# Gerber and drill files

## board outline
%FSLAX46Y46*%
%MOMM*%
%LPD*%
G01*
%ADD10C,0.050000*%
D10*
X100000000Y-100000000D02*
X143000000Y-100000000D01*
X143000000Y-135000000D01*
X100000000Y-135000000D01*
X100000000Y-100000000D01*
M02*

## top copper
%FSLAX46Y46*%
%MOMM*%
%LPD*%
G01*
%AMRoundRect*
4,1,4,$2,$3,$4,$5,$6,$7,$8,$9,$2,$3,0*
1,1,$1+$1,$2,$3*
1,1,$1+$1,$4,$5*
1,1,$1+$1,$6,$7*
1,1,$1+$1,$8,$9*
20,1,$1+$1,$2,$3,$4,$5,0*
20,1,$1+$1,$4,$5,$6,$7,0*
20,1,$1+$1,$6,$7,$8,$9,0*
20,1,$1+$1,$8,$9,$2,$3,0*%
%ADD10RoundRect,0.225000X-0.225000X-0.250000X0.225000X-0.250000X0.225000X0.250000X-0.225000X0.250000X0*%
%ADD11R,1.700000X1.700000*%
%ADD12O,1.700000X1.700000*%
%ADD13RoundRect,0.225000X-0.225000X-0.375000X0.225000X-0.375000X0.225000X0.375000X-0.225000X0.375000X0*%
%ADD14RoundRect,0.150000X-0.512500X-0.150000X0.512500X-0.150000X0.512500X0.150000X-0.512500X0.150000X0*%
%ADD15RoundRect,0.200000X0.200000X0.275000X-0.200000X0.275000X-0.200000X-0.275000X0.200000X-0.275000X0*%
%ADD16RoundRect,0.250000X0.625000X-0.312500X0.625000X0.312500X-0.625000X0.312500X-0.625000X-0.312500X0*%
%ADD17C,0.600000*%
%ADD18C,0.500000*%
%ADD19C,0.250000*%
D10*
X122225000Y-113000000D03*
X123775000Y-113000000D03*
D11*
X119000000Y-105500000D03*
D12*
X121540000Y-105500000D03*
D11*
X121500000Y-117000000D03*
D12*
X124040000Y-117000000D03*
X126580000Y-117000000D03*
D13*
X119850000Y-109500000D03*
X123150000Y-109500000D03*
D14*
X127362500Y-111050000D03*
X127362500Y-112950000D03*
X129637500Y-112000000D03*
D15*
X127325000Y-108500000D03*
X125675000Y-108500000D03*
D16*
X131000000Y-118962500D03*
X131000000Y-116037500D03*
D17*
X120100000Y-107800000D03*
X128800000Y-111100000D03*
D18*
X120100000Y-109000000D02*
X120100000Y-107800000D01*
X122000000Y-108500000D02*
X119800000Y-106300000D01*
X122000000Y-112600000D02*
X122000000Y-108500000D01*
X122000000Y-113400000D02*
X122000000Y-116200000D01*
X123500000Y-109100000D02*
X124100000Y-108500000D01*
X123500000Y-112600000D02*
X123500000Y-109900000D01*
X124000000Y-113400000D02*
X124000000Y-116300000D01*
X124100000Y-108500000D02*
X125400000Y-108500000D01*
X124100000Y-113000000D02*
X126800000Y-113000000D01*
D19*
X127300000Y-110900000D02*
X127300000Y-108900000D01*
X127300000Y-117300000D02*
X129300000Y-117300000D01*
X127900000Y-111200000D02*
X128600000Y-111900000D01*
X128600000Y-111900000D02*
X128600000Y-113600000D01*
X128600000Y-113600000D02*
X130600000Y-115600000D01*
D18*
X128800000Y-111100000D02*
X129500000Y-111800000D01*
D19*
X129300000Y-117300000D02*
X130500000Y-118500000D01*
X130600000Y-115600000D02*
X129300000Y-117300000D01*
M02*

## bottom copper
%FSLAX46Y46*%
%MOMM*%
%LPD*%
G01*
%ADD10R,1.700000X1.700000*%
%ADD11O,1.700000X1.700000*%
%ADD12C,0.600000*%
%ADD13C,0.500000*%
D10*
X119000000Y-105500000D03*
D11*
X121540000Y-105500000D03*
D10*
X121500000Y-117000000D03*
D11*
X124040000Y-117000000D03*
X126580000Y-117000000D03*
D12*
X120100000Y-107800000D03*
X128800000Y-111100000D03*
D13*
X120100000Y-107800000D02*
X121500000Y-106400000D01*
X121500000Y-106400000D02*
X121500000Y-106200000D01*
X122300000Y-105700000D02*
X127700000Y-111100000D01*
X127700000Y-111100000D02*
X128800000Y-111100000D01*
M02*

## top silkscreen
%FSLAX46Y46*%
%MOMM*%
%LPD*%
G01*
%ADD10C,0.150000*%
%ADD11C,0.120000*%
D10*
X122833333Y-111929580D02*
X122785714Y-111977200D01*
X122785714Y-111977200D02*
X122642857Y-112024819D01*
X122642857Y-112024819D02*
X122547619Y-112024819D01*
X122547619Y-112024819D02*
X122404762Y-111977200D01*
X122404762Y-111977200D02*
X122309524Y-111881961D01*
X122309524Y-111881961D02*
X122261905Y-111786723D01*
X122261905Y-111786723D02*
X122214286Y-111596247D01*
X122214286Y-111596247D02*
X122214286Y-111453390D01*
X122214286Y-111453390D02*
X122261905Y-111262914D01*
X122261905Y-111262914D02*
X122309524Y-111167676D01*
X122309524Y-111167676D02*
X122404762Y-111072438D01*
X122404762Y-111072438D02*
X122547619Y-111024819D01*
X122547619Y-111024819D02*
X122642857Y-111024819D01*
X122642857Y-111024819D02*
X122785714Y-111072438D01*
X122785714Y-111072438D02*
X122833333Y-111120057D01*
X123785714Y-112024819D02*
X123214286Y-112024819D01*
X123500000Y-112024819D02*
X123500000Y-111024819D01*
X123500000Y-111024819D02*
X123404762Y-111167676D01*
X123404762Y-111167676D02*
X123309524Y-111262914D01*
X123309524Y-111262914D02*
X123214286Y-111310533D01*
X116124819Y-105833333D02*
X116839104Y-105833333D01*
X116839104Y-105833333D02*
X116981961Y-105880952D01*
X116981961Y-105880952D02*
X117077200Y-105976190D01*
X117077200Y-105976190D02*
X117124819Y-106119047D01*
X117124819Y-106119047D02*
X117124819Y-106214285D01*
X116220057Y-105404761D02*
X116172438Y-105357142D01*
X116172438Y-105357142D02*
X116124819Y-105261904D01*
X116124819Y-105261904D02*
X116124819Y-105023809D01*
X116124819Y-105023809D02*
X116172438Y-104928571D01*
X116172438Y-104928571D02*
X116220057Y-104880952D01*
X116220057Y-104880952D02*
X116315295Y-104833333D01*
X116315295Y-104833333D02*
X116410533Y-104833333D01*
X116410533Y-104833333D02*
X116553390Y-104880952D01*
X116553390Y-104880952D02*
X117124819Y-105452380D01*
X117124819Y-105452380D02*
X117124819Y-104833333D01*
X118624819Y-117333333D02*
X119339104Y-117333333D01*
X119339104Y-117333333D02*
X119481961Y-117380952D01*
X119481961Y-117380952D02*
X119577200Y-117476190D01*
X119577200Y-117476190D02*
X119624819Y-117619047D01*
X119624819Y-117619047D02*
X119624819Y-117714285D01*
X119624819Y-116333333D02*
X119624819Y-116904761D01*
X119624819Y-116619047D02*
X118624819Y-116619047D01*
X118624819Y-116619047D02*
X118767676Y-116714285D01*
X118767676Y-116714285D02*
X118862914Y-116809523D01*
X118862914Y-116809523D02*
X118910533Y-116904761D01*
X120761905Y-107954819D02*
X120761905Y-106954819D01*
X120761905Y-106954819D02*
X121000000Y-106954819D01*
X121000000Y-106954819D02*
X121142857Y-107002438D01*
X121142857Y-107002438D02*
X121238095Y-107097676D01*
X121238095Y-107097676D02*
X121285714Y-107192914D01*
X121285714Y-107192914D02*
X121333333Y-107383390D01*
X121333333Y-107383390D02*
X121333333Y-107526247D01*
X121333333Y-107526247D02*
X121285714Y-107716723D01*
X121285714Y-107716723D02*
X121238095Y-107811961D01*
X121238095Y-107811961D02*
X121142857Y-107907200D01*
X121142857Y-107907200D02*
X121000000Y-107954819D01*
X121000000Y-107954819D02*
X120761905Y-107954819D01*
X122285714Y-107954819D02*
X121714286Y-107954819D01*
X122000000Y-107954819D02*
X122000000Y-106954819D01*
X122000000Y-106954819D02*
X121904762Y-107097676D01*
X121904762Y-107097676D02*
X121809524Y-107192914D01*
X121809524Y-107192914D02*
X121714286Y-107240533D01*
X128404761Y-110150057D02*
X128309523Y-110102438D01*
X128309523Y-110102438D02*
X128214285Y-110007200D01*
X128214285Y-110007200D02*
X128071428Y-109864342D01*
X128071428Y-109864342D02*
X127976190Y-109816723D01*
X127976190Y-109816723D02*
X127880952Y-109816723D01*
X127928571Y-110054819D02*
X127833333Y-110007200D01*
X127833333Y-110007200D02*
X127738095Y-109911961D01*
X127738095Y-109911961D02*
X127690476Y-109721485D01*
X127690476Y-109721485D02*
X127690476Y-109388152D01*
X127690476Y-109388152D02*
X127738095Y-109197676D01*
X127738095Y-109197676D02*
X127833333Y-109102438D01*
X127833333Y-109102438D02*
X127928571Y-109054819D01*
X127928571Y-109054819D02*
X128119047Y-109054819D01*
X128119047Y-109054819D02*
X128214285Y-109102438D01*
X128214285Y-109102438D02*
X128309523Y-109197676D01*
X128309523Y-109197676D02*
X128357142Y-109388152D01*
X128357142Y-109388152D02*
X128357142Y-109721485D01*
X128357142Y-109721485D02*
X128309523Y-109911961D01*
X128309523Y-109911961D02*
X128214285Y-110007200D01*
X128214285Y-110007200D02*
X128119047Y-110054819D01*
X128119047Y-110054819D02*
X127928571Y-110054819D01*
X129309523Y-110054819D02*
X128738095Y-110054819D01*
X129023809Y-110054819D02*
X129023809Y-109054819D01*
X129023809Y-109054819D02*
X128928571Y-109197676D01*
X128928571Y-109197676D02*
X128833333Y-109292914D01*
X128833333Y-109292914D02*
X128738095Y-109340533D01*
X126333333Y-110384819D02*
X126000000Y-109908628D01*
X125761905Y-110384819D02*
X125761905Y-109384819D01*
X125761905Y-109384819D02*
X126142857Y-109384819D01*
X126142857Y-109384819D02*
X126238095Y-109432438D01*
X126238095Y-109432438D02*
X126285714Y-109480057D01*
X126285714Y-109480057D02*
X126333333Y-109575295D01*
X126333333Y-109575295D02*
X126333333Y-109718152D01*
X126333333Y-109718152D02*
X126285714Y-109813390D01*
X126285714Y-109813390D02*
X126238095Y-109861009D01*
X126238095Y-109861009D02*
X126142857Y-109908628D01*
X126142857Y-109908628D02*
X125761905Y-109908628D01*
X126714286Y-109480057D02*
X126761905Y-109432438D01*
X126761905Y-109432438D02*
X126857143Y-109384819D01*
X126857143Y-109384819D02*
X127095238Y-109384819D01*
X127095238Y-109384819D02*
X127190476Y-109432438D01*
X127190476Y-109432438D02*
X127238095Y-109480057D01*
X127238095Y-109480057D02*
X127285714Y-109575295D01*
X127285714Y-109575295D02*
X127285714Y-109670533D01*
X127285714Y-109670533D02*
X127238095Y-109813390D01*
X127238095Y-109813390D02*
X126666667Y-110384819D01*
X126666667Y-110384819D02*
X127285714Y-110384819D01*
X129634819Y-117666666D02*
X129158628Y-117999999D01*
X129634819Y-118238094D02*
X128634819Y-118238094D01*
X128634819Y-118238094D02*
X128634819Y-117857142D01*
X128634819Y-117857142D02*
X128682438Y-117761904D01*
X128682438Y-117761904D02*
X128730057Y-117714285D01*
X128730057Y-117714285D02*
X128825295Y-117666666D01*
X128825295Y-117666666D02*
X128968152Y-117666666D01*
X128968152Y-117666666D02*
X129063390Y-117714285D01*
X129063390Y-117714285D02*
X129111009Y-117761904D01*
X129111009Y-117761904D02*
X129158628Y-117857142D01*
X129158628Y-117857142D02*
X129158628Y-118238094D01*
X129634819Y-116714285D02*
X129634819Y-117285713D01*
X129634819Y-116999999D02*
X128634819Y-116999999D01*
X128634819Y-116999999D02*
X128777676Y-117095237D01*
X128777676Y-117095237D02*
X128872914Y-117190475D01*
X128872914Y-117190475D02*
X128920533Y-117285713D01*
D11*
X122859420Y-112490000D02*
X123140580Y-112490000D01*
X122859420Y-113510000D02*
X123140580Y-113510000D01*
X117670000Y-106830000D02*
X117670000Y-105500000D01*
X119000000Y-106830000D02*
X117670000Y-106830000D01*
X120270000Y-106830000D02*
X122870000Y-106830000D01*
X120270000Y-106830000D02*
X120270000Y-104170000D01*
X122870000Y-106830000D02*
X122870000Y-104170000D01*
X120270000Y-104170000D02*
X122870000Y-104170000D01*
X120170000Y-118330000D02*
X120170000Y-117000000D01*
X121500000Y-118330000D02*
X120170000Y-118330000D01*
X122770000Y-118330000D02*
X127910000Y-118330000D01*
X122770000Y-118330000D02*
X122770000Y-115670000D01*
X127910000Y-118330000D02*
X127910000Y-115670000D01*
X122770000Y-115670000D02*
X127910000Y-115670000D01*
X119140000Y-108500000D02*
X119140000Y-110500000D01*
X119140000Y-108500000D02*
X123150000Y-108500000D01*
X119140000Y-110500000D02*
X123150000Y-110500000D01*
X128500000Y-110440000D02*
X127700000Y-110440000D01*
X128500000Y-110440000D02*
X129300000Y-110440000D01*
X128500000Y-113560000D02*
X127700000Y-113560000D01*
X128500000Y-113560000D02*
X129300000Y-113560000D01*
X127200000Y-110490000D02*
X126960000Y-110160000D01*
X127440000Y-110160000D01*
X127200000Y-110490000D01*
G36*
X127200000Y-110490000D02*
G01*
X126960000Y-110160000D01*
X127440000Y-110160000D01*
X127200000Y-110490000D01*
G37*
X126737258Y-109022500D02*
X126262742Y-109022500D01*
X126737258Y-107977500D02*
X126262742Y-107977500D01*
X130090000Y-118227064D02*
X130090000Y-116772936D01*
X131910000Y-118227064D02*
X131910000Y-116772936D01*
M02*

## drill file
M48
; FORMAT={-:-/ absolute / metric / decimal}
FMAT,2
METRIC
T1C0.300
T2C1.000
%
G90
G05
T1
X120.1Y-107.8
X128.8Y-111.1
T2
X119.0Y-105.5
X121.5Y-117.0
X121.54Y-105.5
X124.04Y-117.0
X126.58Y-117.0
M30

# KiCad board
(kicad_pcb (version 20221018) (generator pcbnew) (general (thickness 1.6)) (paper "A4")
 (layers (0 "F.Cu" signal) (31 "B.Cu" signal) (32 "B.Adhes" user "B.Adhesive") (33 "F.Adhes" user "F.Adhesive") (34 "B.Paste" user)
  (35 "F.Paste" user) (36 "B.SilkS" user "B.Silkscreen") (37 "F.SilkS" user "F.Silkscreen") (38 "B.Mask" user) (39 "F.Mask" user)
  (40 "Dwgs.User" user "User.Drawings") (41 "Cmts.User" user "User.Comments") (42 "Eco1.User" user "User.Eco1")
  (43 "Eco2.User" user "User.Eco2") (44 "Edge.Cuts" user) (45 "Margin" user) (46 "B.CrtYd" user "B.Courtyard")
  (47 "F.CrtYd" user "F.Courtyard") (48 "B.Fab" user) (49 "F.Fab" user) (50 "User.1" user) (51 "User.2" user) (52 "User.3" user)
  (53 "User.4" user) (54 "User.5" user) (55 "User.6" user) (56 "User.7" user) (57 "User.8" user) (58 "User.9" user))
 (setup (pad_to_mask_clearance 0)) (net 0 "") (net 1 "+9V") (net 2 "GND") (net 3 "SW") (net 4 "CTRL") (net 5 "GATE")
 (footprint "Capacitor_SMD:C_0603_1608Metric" (layer "F.Cu") (at 123 113)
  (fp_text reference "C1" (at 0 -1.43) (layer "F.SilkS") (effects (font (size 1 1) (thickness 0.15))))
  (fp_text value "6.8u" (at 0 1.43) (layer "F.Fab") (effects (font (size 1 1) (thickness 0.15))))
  (fp_line (start -0.14058 -0.51) (end 0.14058 -0.51) (stroke (width 0.12) (type solid)) (layer "F.SilkS"))
  (fp_line (start -0.14058 0.51) (end 0.14058 0.51) (stroke (width 0.12) (type solid)) (layer "F.SilkS"))
  (pad "1" smd roundrect (at -0.775 0) (size 0.9 0.95) (layers "F.Cu" "F.Paste" "F.Mask") (roundrect_rratio 0.25) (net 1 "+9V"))
  (pad "2" smd roundrect (at 0.775 0) (size 0.9 0.95) (layers "F.Cu" "F.Paste" "F.Mask") (roundrect_rratio 0.25) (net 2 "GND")))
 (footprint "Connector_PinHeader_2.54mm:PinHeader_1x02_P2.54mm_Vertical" (layer "F.Cu") (at 119 105.5 90)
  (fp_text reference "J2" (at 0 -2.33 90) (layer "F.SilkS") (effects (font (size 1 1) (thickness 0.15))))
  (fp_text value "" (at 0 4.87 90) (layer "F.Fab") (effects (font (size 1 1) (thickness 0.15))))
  (fp_line (start -1.33 -1.33) (end 0 -1.33) (stroke (width 0.12) (type solid)) (layer "F.SilkS"))
  (fp_line (start -1.33 0) (end -1.33 -1.33) (stroke (width 0.12) (type solid)) (layer "F.SilkS"))
  (fp_line (start -1.33 1.27) (end -1.33 3.87) (stroke (width 0.12) (type solid)) (layer "F.SilkS"))
  (fp_line (start -1.33 1.27) (end 1.33 1.27) (stroke (width 0.12) (type solid)) (layer "F.SilkS"))
  (fp_line (start -1.33 3.87) (end 1.33 3.87) (stroke (width 0.12) (type solid)) (layer "F.SilkS"))
  (fp_line (start 1.33 1.27) (end 1.33 3.87) (stroke (width 0.12) (type solid)) (layer "F.SilkS"))
  (pad "1" thru_hole rect (at 0 0 90) (size 1.7 1.7) (drill 1) (layers "*.Cu" "*.Mask") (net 1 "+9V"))
  (pad "2" thru_hole oval (at 0 2.54 90) (size 1.7 1.7) (drill 1) (layers "*.Cu" "*.Mask") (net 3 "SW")))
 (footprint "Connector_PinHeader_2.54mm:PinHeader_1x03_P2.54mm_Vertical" (layer "F.Cu") (at 121.5 117 90)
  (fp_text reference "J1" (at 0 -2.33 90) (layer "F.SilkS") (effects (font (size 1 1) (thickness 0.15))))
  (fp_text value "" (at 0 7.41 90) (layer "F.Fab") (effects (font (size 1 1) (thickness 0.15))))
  (fp_line (start -1.33 -1.33) (end 0 -1.33) (stroke (width 0.12) (type solid)) (layer "F.SilkS"))
  (fp_line (start -1.33 0) (end -1.33 -1.33) (stroke (width 0.12) (type solid)) (layer "F.SilkS"))
  (fp_line (start -1.33 1.27) (end -1.33 6.41) (stroke (width 0.12) (type solid)) (layer "F.SilkS"))
  (fp_line (start -1.33 1.27) (end 1.33 1.27) (stroke (width 0.12) (type solid)) (layer "F.SilkS"))
  (fp_line (start -1.33 6.41) (end 1.33 6.41) (stroke (width 0.12) (type solid)) (layer "F.SilkS"))
  (fp_line (start 1.33 1.27) (end 1.33 6.41) (stroke (width 0.12) (type solid)) (layer "F.SilkS"))
  (pad "1" thru_hole rect (at 0 0 90) (size 1.7 1.7) (drill 1) (layers "*.Cu" "*.Mask") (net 1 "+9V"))
  (pad "2" thru_hole oval (at 0 2.54 90) (size 1.7 1.7) (drill 1) (layers "*.Cu" "*.Mask") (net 2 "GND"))
  (pad "3" thru_hole oval (at 0 5.08 90) (size 1.7 1.7) (drill 1) (layers "*.Cu" "*.Mask") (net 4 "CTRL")))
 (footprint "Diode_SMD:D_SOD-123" (layer "F.Cu") (at 121.5 109.5)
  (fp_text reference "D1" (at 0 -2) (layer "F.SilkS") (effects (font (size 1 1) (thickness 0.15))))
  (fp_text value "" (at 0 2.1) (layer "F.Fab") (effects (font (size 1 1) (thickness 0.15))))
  (fp_line (start -2.36 -1) (end -2.36 1) (stroke (width 0.12) (type solid)) (layer "F.SilkS"))
  (fp_line (start -2.36 -1) (end 1.65 -1) (stroke (width 0.12) (type solid)) (layer "F.SilkS"))
  (fp_line (start -2.36 1) (end 1.65 1) (stroke (width 0.12) (type solid)) (layer "F.SilkS"))
  (pad "1" smd roundrect (at -1.65 0) (size 0.9 1.2) (layers "F.Cu" "F.Paste" "F.Mask") (roundrect_rratio 0.25) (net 3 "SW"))
  (pad "2" smd roundrect (at 1.65 0) (size 0.9 1.2) (layers "F.Cu" "F.Paste" "F.Mask") (roundrect_rratio 0.25) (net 2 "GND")))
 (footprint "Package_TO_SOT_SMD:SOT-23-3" (layer "F.Cu") (at 128.5 112)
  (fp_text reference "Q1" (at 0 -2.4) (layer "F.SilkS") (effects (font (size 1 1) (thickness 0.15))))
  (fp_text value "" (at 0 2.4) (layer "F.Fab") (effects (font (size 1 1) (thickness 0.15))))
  (fp_line (start 0 -1.56) (end -0.8 -1.56) (stroke (width 0.12) (type solid)) (layer "F.SilkS"))
  (fp_line (start 0 -1.56) (end 0.8 -1.56) (stroke (width 0.12) (type solid)) (layer "F.SilkS"))
  (fp_line (start 0 1.56) (end -0.8 1.56) (stroke (width 0.12) (type solid)) (layer "F.SilkS"))
  (fp_line (start 0 1.56) (end 0.8 1.56) (stroke (width 0.12) (type solid)) (layer "F.SilkS"))
  (fp_poly
   (pts (xy -1.3 -1.51) (xy -1.54 -1.84) (xy -1.06 -1.84) (xy -1.3 -1.51)) (stroke (width 0.12) (type solid)) (fill solid) (layer "F.SilkS"))
  (pad "1" smd roundrect (at -1.1375 -0.95) (size 1.325 0.6) (layers "F.Cu" "F.Paste" "F.Mask") (roundrect_rratio 0.25) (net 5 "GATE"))
  (pad "2" smd roundrect (at -1.1375 0.95) (size 1.325 0.6) (layers "F.Cu" "F.Paste" "F.Mask") (roundrect_rratio 0.25) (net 2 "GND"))
  (pad "3" smd roundrect (at 1.1375 0) (size 1.325 0.6) (layers "F.Cu" "F.Paste" "F.Mask") (roundrect_rratio 0.25) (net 3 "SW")))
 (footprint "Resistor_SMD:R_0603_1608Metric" (layer "F.Cu") (at 126.5 108.5 180)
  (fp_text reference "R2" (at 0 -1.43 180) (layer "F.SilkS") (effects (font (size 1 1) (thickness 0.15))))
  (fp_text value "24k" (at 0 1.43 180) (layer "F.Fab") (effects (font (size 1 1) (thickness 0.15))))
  (fp_line (start -0.237258 -0.5225) (end 0.237258 -0.5225) (stroke (width 0.12) (type solid)) (layer "F.SilkS"))
  (fp_line (start -0.237258 0.5225) (end 0.237258 0.5225) (stroke (width 0.12) (type solid)) (layer "F.SilkS"))
  (pad "1" smd roundrect (at -0.825 0 180) (size 0.8 0.95) (layers "F.Cu" "F.Paste" "F.Mask") (roundrect_rratio 0.25) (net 5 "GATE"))
  (pad "2" smd roundrect (at 0.825 0 180) (size 0.8 0.95) (layers "F.Cu" "F.Paste" "F.Mask") (roundrect_rratio 0.25) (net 2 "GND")))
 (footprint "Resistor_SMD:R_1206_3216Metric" (layer "F.Cu") (at 131 117.5 90)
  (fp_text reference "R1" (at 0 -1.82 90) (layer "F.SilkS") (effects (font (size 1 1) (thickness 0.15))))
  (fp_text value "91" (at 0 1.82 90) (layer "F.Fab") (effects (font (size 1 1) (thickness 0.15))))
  (fp_line (start -0.727064 -0.91) (end 0.727064 -0.91) (stroke (width 0.12) (type solid)) (layer "F.SilkS"))
  (fp_line (start -0.727064 0.91) (end 0.727064 0.91) (stroke (width 0.12) (type solid)) (layer "F.SilkS"))
  (pad "1" smd roundrect (at -1.4625 0 90) (size 1.125 1.75) (layers "F.Cu" "F.Paste" "F.Mask") (roundrect_rratio 0.222222) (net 4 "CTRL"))
  (pad "2" smd roundrect (at 1.4625 0 90) (size 1.125 1.75) (layers "F.Cu" "F.Paste" "F.Mask") (roundrect_rratio 0.222222) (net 5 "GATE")))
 (gr_rect (start 100 100) (end 143 135) (stroke (width 0.05) (type default)) (fill none) (layer "Edge.Cuts"))
 (segment (start 120.1 109) (end 120.1 107.8) (width 0.5) (layer "F.Cu") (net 3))
 (segment (start 122 108.5) (end 119.8 106.3) (width 0.5) (layer "F.Cu") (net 1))
 (segment (start 122 112.6) (end 122 108.5) (width 0.5) (layer "F.Cu") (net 1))
 (segment (start 122 113.4) (end 122 116.2) (width 0.5) (layer "F.Cu") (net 1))
 (segment (start 123.5 109.1) (end 124.1 108.5) (width 0.5) (layer "F.Cu") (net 2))
 (segment (start 123.5 112.6) (end 123.5 109.9) (width 0.5) (layer "F.Cu") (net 2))
 (segment (start 124 113.4) (end 124 116.3) (width 0.5) (layer "F.Cu") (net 2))
 (segment (start 124.1 108.5) (end 125.4 108.5) (width 0.5) (layer "F.Cu") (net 2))
 (segment (start 124.1 113) (end 126.8 113) (width 0.5) (layer "F.Cu") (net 2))
 (segment (start 127.3 110.9) (end 127.3 108.9) (width 0.25) (layer "F.Cu") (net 5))
 (segment (start 127.3 117.3) (end 129.3 117.3) (width 0.25) (layer "F.Cu") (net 4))
 (segment (start 127.9 111.2) (end 128.6 111.9) (width 0.25) (layer "F.Cu") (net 5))
 (segment (start 128.6 111.9) (end 128.6 113.6) (width 0.25) (layer "F.Cu") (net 5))
 (segment (start 128.6 113.6) (end 130.6 115.6) (width 0.25) (layer "F.Cu") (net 5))
 (segment (start 128.8 111.1) (end 129.5 111.8) (width 0.5) (layer "F.Cu") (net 3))
 (segment (start 129.3 117.3) (end 130.5 118.5) (width 0.25) (layer "F.Cu") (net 4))
 (segment (start 130.6 115.6) (end 129.3 117.3) (width 0.25) (layer "F.Cu") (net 5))
 (via (at 120.1 107.8) (size 0.6) (drill 0.3) (layers "F.Cu" "B.Cu") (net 3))
 (via (at 128.8 111.1) (size 0.6) (drill 0.3) (layers "F.Cu" "B.Cu") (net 3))
 (segment (start 120.1 107.8) (end 121.5 106.4) (width 0.5) (layer "B.Cu") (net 3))
 (segment (start 121.5 106.4) (end 121.5 106.2) (width 0.5) (layer "B.Cu") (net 3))
 (segment (start 122.3 105.7) (end 127.7 111.1) (width 0.5) (layer "B.Cu") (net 3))
 (segment (start 127.7 111.1) (end 128.8 111.1) (width 0.5) (layer "B.Cu") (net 3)))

